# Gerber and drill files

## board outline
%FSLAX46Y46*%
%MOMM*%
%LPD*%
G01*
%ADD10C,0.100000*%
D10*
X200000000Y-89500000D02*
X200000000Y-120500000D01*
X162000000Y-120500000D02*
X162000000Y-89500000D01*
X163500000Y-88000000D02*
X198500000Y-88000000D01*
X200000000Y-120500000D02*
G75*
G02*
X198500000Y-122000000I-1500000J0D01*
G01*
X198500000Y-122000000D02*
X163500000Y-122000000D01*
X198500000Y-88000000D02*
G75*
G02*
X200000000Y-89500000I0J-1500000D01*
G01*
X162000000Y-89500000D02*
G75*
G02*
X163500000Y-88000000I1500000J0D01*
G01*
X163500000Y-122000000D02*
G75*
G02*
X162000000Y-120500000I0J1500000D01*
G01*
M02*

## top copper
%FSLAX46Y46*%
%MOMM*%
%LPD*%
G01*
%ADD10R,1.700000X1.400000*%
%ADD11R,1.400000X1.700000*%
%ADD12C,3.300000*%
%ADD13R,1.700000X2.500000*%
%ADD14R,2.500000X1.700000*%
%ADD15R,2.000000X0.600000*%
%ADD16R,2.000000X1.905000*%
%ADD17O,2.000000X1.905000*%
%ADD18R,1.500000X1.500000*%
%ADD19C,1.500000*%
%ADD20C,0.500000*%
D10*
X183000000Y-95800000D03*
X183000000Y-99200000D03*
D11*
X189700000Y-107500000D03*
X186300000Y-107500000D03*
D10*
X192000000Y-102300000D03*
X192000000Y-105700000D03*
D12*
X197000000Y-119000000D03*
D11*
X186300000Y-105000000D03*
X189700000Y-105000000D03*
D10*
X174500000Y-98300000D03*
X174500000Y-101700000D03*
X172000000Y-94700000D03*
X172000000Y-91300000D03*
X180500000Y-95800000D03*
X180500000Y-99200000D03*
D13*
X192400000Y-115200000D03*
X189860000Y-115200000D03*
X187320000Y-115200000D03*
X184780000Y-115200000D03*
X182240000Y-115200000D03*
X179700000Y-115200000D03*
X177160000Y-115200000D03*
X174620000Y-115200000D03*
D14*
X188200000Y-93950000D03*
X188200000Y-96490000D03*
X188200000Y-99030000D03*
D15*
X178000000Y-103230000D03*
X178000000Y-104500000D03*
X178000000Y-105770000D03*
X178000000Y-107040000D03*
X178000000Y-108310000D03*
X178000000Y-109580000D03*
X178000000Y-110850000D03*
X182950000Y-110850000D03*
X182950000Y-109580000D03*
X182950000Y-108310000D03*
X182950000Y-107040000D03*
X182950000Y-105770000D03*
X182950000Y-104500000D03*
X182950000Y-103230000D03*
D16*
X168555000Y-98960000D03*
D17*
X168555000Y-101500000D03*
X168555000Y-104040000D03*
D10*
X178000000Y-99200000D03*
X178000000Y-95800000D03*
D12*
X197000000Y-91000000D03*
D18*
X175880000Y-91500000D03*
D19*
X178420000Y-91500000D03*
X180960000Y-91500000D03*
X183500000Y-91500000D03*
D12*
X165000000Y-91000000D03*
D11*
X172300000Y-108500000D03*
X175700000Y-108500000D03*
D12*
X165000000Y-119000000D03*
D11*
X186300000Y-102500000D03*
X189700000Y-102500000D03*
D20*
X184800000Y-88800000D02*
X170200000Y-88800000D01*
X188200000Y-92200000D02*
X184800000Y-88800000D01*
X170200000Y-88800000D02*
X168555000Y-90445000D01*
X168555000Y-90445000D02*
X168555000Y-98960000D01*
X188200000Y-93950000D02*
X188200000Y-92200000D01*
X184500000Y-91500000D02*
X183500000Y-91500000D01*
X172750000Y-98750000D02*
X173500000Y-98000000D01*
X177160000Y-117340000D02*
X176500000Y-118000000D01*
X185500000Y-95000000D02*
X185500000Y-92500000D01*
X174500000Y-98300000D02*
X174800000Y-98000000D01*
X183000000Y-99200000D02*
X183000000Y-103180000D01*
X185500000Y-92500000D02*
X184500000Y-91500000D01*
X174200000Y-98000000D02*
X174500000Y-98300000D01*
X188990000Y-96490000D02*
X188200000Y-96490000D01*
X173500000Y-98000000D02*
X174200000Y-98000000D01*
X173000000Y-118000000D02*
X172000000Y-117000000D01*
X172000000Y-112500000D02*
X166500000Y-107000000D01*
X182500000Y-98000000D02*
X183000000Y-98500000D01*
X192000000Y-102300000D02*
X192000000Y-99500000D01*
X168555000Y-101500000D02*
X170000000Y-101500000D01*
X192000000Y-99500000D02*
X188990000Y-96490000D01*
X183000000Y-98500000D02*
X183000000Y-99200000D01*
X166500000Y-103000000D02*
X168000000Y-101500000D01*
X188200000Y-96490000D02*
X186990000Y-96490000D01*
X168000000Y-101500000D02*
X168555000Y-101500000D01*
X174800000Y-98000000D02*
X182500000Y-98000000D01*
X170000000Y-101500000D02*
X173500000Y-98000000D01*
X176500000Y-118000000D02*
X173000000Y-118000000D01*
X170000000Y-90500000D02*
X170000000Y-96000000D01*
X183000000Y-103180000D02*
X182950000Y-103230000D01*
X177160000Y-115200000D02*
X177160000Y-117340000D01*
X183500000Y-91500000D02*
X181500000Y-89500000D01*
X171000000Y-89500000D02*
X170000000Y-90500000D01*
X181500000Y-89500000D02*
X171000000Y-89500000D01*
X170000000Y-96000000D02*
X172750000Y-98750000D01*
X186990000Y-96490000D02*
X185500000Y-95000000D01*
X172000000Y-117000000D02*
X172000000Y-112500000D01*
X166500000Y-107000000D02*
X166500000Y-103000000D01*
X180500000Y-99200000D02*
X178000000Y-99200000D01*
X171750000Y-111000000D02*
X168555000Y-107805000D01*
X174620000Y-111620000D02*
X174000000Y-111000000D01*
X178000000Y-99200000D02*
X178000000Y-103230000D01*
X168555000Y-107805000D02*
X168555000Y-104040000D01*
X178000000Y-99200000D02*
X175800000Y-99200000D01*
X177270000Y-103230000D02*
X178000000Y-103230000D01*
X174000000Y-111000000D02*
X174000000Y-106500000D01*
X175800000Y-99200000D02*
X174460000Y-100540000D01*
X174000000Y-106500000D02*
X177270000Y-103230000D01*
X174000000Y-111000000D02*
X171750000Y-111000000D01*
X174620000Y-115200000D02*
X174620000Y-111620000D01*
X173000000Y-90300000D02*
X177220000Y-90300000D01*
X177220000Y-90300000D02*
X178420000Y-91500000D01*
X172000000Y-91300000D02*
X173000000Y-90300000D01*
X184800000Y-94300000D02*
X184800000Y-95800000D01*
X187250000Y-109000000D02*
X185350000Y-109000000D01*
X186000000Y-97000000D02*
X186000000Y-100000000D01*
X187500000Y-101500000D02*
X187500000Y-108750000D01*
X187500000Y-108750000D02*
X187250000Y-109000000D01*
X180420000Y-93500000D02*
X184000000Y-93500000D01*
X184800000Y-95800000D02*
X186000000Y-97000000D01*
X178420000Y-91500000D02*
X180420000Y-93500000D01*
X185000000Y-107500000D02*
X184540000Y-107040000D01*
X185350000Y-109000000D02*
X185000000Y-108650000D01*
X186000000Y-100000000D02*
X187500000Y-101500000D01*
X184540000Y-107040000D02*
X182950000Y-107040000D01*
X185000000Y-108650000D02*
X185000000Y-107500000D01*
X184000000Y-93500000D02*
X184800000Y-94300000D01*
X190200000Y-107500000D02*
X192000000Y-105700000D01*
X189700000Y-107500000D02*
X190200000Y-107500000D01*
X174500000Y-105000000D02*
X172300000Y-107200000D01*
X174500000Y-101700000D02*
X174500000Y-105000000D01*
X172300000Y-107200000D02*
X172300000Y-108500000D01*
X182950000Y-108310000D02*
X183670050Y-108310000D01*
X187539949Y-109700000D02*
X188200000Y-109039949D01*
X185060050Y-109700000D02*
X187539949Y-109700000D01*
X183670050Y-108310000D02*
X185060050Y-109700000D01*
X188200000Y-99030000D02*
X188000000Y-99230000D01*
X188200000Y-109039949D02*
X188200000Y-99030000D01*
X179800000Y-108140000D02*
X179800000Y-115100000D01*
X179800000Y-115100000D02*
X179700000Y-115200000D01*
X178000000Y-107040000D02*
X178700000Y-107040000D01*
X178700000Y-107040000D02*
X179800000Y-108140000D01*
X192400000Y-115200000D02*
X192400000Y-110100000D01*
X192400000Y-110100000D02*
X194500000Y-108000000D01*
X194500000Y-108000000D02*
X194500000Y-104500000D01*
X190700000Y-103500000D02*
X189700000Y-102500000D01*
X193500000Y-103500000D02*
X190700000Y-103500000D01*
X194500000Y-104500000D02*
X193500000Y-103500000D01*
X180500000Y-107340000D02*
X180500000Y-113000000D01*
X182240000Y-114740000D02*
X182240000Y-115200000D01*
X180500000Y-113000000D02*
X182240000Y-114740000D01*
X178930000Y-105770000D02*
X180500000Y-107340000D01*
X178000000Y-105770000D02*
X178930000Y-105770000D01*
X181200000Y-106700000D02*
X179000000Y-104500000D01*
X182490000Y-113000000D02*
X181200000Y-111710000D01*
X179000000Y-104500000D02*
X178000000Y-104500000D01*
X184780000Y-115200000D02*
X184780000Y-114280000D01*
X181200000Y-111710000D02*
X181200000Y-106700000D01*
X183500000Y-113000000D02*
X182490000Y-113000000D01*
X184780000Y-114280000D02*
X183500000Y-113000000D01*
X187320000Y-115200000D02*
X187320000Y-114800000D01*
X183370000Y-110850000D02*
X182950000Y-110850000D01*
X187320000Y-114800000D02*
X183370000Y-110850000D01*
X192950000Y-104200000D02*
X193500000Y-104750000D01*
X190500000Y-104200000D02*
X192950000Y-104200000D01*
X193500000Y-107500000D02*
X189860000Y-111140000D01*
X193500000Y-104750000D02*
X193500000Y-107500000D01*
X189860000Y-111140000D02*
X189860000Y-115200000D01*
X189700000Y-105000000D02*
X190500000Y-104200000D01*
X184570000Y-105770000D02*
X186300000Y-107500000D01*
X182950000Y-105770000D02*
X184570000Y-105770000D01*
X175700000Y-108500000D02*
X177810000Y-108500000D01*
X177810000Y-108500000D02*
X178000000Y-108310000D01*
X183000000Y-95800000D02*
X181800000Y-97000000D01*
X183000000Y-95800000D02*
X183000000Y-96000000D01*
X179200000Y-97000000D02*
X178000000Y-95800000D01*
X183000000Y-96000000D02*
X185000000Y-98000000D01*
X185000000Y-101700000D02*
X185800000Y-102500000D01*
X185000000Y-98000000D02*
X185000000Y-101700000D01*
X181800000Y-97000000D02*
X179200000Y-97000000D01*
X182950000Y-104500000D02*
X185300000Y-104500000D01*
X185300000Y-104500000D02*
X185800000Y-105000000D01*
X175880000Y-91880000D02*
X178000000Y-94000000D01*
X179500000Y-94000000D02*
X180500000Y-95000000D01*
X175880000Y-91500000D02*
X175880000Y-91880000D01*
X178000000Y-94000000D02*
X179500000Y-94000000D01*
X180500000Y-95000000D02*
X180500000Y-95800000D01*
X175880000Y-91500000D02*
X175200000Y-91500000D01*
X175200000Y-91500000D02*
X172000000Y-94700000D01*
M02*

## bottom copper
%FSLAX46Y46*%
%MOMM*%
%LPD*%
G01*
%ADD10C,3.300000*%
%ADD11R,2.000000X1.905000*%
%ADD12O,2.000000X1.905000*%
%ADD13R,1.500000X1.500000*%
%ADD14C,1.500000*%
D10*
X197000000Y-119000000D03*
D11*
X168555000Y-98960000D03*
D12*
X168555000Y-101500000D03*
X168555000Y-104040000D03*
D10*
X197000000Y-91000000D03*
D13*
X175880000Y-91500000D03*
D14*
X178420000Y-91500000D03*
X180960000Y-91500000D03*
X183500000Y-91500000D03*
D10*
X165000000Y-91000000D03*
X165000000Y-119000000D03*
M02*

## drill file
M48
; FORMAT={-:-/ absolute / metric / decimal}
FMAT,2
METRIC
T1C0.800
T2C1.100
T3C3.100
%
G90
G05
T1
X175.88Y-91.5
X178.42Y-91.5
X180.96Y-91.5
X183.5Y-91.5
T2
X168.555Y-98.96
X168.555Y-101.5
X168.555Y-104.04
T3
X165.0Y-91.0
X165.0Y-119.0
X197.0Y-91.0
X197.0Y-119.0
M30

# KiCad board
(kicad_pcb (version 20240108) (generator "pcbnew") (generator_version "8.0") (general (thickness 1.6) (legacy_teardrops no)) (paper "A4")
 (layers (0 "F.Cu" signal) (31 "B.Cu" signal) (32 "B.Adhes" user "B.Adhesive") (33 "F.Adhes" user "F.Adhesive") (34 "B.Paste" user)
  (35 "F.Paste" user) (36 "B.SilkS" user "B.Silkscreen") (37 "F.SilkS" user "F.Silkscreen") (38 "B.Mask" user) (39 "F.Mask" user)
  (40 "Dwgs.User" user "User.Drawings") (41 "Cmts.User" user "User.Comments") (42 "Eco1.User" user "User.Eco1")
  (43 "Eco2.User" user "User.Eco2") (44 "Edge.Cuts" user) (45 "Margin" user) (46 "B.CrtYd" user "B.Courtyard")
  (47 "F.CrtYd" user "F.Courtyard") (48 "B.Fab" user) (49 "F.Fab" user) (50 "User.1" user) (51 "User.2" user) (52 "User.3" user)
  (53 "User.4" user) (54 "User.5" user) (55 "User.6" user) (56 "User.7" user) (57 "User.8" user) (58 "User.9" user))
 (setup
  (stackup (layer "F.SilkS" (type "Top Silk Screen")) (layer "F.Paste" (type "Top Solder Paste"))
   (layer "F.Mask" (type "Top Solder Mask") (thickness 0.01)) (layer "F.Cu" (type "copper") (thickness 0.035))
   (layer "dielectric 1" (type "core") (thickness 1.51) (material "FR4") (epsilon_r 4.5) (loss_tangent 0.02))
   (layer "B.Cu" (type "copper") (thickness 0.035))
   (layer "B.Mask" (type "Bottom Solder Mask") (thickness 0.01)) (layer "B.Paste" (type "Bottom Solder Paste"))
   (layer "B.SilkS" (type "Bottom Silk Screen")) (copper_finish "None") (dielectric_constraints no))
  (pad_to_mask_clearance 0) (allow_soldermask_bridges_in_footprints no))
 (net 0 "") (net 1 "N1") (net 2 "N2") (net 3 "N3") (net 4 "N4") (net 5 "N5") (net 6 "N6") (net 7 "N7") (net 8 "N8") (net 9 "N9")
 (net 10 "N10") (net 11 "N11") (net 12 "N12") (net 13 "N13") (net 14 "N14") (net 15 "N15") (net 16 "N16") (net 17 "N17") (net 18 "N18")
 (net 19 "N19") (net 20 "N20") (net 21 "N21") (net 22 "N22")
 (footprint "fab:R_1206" (layer "F.Cu") (at 183 97.5 -90)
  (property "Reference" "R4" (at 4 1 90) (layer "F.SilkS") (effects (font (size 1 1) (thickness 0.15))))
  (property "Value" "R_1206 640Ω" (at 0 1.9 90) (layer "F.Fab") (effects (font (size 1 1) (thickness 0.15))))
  (pad "1" smd rect (at -1.7 0 270) (size 1.4 1.7) (layers "F.Cu" "F.Paste" "F.Mask") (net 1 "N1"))
  (pad "2" smd rect (at 1.7 0 270) (size 1.4 1.7) (layers "F.Cu" "F.Paste" "F.Mask") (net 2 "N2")))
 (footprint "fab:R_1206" (layer "F.Cu") (at 188 107.5 180)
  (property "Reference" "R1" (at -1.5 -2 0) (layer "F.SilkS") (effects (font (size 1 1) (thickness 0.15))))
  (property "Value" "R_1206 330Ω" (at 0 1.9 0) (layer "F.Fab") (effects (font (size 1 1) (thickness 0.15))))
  (pad "1" smd rect (at -1.7 0 180) (size 1.4 1.7) (layers "F.Cu" "F.Paste" "F.Mask") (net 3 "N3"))
  (pad "2" smd rect (at 1.7 0 180) (size 1.4 1.7) (layers "F.Cu" "F.Paste" "F.Mask") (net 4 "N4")))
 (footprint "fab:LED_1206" (layer "F.Cu") (at 192 104 -90)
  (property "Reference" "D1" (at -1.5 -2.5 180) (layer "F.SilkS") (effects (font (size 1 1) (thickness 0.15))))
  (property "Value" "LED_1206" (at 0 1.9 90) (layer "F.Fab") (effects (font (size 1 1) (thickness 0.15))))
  (pad "1" smd rect (at -1.7 0 270) (size 1.4 1.7) (layers "F.Cu" "F.Paste" "F.Mask") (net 2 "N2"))
  (pad "2" smd rect (at 1.7 0 270) (size 1.4 1.7) (layers "F.Cu" "F.Paste" "F.Mask") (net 3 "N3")))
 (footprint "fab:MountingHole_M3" (layer "F.Cu") (at 197 119)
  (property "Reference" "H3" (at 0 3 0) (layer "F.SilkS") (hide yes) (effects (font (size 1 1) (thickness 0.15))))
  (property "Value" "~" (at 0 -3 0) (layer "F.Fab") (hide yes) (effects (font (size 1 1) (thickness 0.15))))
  (pad "" thru_hole circle (at 0 0) (size 3.3 3.3) (drill 3.1) (layers "*.Cu" "*.Mask") (remove_unused_layers no)))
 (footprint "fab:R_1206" (layer "F.Cu") (at 188 105)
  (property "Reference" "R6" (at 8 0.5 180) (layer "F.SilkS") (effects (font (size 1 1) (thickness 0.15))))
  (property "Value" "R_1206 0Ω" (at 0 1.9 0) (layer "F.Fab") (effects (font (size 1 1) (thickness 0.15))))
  (pad "1" smd rect (at -1.7 0) (size 1.4 1.7) (layers "F.Cu" "F.Paste" "F.Mask") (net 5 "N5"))
  (pad "2" smd rect (at 1.7 0) (size 1.4 1.7) (layers "F.Cu" "F.Paste" "F.Mask") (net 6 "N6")))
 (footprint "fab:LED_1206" (layer "F.Cu") (at 174.5 100 -90)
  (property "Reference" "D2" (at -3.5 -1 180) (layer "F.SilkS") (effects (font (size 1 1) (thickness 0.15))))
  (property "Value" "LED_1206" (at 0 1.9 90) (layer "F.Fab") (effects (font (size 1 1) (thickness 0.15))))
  (pad "1" smd rect (at -1.7 0 270) (size 1.4 1.7) (layers "F.Cu" "F.Paste" "F.Mask") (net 2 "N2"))
  (pad "2" smd rect (at 1.7 0 270) (size 1.4 1.7) (layers "F.Cu" "F.Paste" "F.Mask") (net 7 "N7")))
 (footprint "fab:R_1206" (layer "F.Cu") (at 172 93 90)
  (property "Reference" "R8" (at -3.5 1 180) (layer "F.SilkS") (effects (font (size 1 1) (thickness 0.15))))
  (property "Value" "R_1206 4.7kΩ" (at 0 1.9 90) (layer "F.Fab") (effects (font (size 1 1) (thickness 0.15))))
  (pad "1" smd rect (at -1.7 0 90) (size 1.4 1.7) (layers "F.Cu" "F.Paste" "F.Mask") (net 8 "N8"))
  (pad "2" smd rect (at 1.7 0 90) (size 1.4 1.7) (layers "F.Cu" "F.Paste" "F.Mask") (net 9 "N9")))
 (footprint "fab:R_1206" (layer "F.Cu") (at 180.5 97.5 -90)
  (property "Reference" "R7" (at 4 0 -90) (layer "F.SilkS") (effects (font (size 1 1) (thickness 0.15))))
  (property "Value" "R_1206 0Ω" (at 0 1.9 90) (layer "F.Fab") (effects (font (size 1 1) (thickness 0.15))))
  (pad "1" smd rect (at -1.7 0 270) (size 1.4 1.7) (layers "F.Cu" "F.Paste" "F.Mask") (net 8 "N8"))
  (pad "2" smd rect (at 1.7 0 270) (size 1.4 1.7) (layers "F.Cu" "F.Paste" "F.Mask") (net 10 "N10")))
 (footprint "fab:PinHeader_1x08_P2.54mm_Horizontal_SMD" (layer "F.Cu") (at 192.4 115.2 -90)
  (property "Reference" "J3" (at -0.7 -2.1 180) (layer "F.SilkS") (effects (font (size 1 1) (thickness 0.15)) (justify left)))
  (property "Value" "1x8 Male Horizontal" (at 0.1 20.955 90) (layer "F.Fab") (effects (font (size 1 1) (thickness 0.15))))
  (pad "1" smd rect (at 0 0 270) (size 2.5 1.7) (layers "F.Cu" "F.Paste" "F.Mask") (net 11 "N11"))
  (pad "2" smd rect (at 0 2.54 270) (size 2.5 1.7) (layers "F.Cu" "F.Paste" "F.Mask") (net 6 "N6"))
  (pad "3" smd rect (at 0 5.08 270) (size 2.5 1.7) (layers "F.Cu" "F.Paste" "F.Mask") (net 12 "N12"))
  (pad "4" smd rect (at 0 7.62 270) (size 2.5 1.7) (layers "F.Cu" "F.Paste" "F.Mask") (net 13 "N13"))
  (pad "5" smd rect (at 0 10.16 270) (size 2.5 1.7) (layers "F.Cu" "F.Paste" "F.Mask") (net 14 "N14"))
  (pad "6" smd rect (at 0 12.7 270) (size 2.5 1.7) (layers "F.Cu" "F.Paste" "F.Mask") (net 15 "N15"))
  (pad "7" smd rect (at 0 15.24 270) (size 2.5 1.7) (layers "F.Cu" "F.Paste" "F.Mask") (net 2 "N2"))
  (pad "8" smd rect (at 0 17.78 270) (size 2.5 1.7) (layers "F.Cu" "F.Paste" "F.Mask") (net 10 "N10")))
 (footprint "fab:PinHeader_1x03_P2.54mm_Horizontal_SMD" (layer "F.Cu") (at 188.2 93.95)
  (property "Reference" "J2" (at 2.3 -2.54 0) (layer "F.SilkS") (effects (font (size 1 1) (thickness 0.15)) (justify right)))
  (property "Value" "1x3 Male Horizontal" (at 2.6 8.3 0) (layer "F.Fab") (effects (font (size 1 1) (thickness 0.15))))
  (pad "1" smd rect (at 0 0) (size 2.5 1.7) (layers "F.Cu" "F.Paste" "F.Mask") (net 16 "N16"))
  (pad "2" smd rect (at 0 2.54) (size 2.5 1.7) (layers "F.Cu" "F.Paste" "F.Mask") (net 2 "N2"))
  (pad "3" smd rect (at 0 5.08) (size 2.5 1.7) (layers "F.Cu" "F.Paste" "F.Mask") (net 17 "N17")))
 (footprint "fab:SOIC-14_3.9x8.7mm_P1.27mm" (layer "F.Cu") (at 180.475 107.04)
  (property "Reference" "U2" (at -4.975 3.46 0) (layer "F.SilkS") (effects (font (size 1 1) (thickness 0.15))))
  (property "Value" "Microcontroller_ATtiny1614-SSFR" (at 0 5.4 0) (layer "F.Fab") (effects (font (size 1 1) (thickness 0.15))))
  (pad "1" smd rect (at -2.475 -3.81) (size 2 0.6) (layers "F.Cu" "F.Paste" "F.Mask") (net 10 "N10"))
  (pad "2" smd rect (at -2.475 -2.54) (size 2 0.6) (layers "F.Cu" "F.Paste" "F.Mask") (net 13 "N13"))
  (pad "3" smd rect (at -2.475 -1.27) (size 2 0.6) (layers "F.Cu" "F.Paste" "F.Mask") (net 14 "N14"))
  (pad "4" smd rect (at -2.475 0) (size 2 0.6) (layers "F.Cu" "F.Paste" "F.Mask") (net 15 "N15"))
  (pad "5" smd rect (at -2.475 1.27) (size 2 0.6) (layers "F.Cu" "F.Paste" "F.Mask") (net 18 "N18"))
  (pad "6" smd rect (at -2.475 2.54) (size 2 0.6) (layers "F.Cu" "F.Paste" "F.Mask") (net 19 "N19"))
  (pad "7" smd rect (at -2.475 3.81) (size 2 0.6) (layers "F.Cu" "F.Paste" "F.Mask") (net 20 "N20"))
  (pad "8" smd rect (at 2.475 3.81) (size 2 0.6) (layers "F.Cu" "F.Paste" "F.Mask") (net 12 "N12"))
  (pad "9" smd rect (at 2.475 2.54) (size 2 0.6) (layers "F.Cu" "F.Paste" "F.Mask") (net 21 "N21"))
  (pad "10" smd rect (at 2.475 1.27) (size 2 0.6) (layers "F.Cu" "F.Paste" "F.Mask") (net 17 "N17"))
  (pad "11" smd rect (at 2.475 0) (size 2 0.6) (layers "F.Cu" "F.Paste" "F.Mask") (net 9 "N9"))
  (pad "12" smd rect (at 2.475 -1.27) (size 2 0.6) (layers "F.Cu" "F.Paste" "F.Mask") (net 4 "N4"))
  (pad "13" smd rect (at 2.475 -2.54) (size 2 0.6) (layers "F.Cu" "F.Paste" "F.Mask") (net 5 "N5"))
  (pad "14" smd rect (at 2.475 -3.81) (size 2 0.6) (layers "F.Cu" "F.Paste" "F.Mask") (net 2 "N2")))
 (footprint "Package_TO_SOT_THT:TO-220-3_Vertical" (layer "F.Cu") (at 168.555 98.96 -90)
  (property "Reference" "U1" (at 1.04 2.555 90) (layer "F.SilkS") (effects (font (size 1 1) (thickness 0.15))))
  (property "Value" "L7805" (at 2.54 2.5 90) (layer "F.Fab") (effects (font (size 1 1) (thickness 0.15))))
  (pad "1" thru_hole rect (at 0 0 270) (size 1.905 2) (drill 1.1) (layers "*.Cu" "*.Mask") (remove_unused_layers no) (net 16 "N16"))
  (pad "2" thru_hole oval (at 2.54 0 270) (size 1.905 2) (drill 1.1) (layers "*.Cu" "*.Mask") (remove_unused_layers no) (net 2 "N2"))
  (pad "3" thru_hole oval (at 5.08 0 270) (size 1.905 2) (drill 1.1) (layers "*.Cu" "*.Mask") (remove_unused_layers no) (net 10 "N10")))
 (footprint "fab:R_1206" (layer "F.Cu") (at 178 97.5 90)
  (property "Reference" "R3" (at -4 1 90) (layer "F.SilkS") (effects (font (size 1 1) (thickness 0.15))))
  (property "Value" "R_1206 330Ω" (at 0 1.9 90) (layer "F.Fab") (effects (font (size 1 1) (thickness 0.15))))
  (pad "1" smd rect (at -1.7 0 90) (size 1.4 1.7) (layers "F.Cu" "F.Paste" "F.Mask") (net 10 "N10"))
  (pad "2" smd rect (at 1.7 0 90) (size 1.4 1.7) (layers "F.Cu" "F.Paste" "F.Mask") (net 1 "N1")))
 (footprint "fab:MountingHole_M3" (layer "F.Cu") (at 197 91)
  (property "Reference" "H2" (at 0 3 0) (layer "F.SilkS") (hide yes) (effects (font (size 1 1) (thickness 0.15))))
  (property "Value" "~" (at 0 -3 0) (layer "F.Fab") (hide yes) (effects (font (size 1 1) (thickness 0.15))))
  (pad "" thru_hole circle (at 0 0) (size 3.3 3.3) (drill 3.1) (layers "*.Cu" "*.Mask") (remove_unused_layers no)))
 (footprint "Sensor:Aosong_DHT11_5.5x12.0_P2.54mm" (layer "F.Cu") (at 175.88 91.5 90)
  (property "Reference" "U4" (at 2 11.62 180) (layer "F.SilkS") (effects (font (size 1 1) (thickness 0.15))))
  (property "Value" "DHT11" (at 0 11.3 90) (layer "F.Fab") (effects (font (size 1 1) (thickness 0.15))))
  (pad "1" thru_hole rect (at 0 0 90) (size 1.5 1.5) (drill 0.8) (layers "*.Cu" "*.Mask") (remove_unused_layers no) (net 8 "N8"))
  (pad "2" thru_hole circle (at 0 2.54 90) (size 1.5 1.5) (drill 0.8) (layers "*.Cu" "*.Mask") (remove_unused_layers no) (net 9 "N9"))
  (pad "3" thru_hole circle (at 0 5.08 90) (size 1.5 1.5) (drill 0.8) (layers "*.Cu" "*.Mask") (remove_unused_layers no) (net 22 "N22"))
  (pad "4" thru_hole circle (at 0 7.62 90) (size 1.5 1.5) (drill 0.8) (layers "*.Cu" "*.Mask") (remove_unused_layers no) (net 2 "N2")))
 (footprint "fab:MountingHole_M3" (layer "F.Cu") (at 165 91)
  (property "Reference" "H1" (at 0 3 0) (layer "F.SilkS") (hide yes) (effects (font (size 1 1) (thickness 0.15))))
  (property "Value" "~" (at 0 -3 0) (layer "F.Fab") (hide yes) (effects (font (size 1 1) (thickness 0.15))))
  (pad "" thru_hole circle (at 0 0) (size 3.3 3.3) (drill 3.1) (layers "*.Cu" "*.Mask") (remove_unused_layers no)))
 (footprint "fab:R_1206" (layer "F.Cu") (at 174 108.5)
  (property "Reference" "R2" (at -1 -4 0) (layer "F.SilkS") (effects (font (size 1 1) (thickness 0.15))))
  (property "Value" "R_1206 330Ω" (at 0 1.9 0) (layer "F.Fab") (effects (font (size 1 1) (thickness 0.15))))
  (pad "1" smd rect (at -1.7 0) (size 1.4 1.7) (layers "F.Cu" "F.Paste" "F.Mask") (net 7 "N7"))
  (pad "2" smd rect (at 1.7 0) (size 1.4 1.7) (layers "F.Cu" "F.Paste" "F.Mask") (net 18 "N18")))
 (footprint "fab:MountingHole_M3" (layer "F.Cu") (at 165 119)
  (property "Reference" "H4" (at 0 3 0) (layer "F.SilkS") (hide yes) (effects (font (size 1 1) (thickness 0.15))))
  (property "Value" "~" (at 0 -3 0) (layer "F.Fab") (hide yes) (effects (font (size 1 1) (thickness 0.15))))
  (pad "" thru_hole circle (at 0 0) (size 3.3 3.3) (drill 3.1) (layers "*.Cu" "*.Mask") (remove_unused_layers no)))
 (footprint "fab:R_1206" (layer "F.Cu") (at 188 102.5)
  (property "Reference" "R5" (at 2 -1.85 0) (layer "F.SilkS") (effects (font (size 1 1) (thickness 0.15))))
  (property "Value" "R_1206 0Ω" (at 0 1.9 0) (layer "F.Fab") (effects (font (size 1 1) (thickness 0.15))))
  (pad "1" smd rect (at -1.7 0) (size 1.4 1.7) (layers "F.Cu" "F.Paste" "F.Mask") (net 1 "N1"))
  (pad "2" smd rect (at 1.7 0) (size 1.4 1.7) (layers "F.Cu" "F.Paste" "F.Mask") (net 11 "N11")))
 (gr_line (start 200 89.5) (end 200 120.5) (stroke (width 0.1) (type default)) (layer "Edge.Cuts"))
 (gr_line (start 162 120.5) (end 162 89.5) (stroke (width 0.1) (type default)) (layer "Edge.Cuts"))
 (gr_line (start 163.5 88) (end 198.5 88) (stroke (width 0.1) (type default)) (layer "Edge.Cuts"))
 (gr_arc (start 200 120.5) (mid 199.56066 121.56066) (end 198.5 122) (stroke (width 0.1) (type default)) (layer "Edge.Cuts"))
 (gr_line (start 198.5 122) (end 163.5 122) (stroke (width 0.1) (type default)) (layer "Edge.Cuts"))
 (gr_arc (start 198.5 88) (mid 199.56066 88.43934) (end 200 89.5) (stroke (width 0.1) (type default)) (layer "Edge.Cuts"))
 (gr_arc (start 162 89.5) (mid 162.43934 88.43934) (end 163.5 88) (stroke (width 0.1) (type default)) (layer "Edge.Cuts"))
 (gr_arc (start 163.5 122) (mid 162.43934 121.56066) (end 162 120.5) (stroke (width 0.1) (type default)) (layer "Edge.Cuts"))
 (segment (start 184.8 88.8) (end 170.2 88.8) (width 0.5) (layer "F.Cu") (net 16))
 (segment (start 188.2 92.2) (end 184.8 88.8) (width 0.5) (layer "F.Cu") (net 16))
 (segment (start 170.2 88.8) (end 168.555 90.445) (width 0.5) (layer "F.Cu") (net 16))
 (segment (start 168.555 90.445) (end 168.555 98.96) (width 0.5) (layer "F.Cu") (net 16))
 (segment (start 188.2 93.95) (end 188.2 92.2) (width 0.5) (layer "F.Cu") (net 16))
 (segment (start 184.5 91.5) (end 183.5 91.5) (width 0.5) (layer "F.Cu") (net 2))
 (segment (start 172.75 98.75) (end 173.5 98) (width 0.5) (layer "F.Cu") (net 2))
 (segment (start 177.16 117.34) (end 176.5 118) (width 0.5) (layer "F.Cu") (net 2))
 (segment (start 185.5 95) (end 185.5 92.5) (width 0.5) (layer "F.Cu") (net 2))
 (segment (start 174.5 98.3) (end 174.8 98) (width 0.5) (layer "F.Cu") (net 2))
 (segment (start 183 99.2) (end 183 103.18) (width 0.5) (layer "F.Cu") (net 2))
 (segment (start 185.5 92.5) (end 184.5 91.5) (width 0.5) (layer "F.Cu") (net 2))
 (segment (start 174.2 98) (end 174.5 98.3) (width 0.5) (layer "F.Cu") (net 2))
 (segment (start 188.99 96.49) (end 188.2 96.49) (width 0.5) (layer "F.Cu") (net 2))
 (segment (start 173.5 98) (end 174.2 98) (width 0.5) (layer "F.Cu") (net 2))
 (segment (start 173 118) (end 172 117) (width 0.5) (layer "F.Cu") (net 2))
 (segment (start 172 112.5) (end 166.5 107) (width 0.5) (layer "F.Cu") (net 2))
 (segment (start 182.5 98) (end 183 98.5) (width 0.5) (layer "F.Cu") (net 2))
 (segment (start 192 102.3) (end 192 99.5) (width 0.5) (layer "F.Cu") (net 2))
 (segment (start 168.555 101.5) (end 170 101.5) (width 0.5) (layer "F.Cu") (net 2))
 (segment (start 192 99.5) (end 188.99 96.49) (width 0.5) (layer "F.Cu") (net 2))
 (segment (start 183 98.5) (end 183 99.2) (width 0.5) (layer "F.Cu") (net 2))
 (segment (start 166.5 103) (end 168 101.5) (width 0.5) (layer "F.Cu") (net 2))
 (segment (start 188.2 96.49) (end 186.99 96.49) (width 0.5) (layer "F.Cu") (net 2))
 (segment (start 168 101.5) (end 168.555 101.5) (width 0.5) (layer "F.Cu") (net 2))
 (segment (start 174.8 98) (end 182.5 98) (width 0.5) (layer "F.Cu") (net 2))
 (segment (start 170 101.5) (end 173.5 98) (width 0.5) (layer "F.Cu") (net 2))
 (segment (start 176.5 118) (end 173 118) (width 0.5) (layer "F.Cu") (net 2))
 (segment (start 170 90.5) (end 170 96) (width 0.5) (layer "F.Cu") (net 2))
 (segment (start 183 103.18) (end 182.95 103.23) (width 0.5) (layer "F.Cu") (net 2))
 (segment (start 177.16 115.2) (end 177.16 117.34) (width 0.5) (layer "F.Cu") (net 2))
 (segment (start 183.5 91.5) (end 181.5 89.5) (width 0.5) (layer "F.Cu") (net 2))
 (segment (start 171 89.5) (end 170 90.5) (width 0.5) (layer "F.Cu") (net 2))
 (segment (start 181.5 89.5) (end 171 89.5) (width 0.5) (layer "F.Cu") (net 2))
 (segment (start 170 96) (end 172.75 98.75) (width 0.5) (layer "F.Cu") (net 2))
 (segment (start 186.99 96.49) (end 185.5 95) (width 0.5) (layer "F.Cu") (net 2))
 (segment (start 172 117) (end 172 112.5) (width 0.5) (layer "F.Cu") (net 2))
 (segment (start 166.5 107) (end 166.5 103) (width 0.5) (layer "F.Cu") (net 2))
 (segment (start 180.5 99.2) (end 178 99.2) (width 0.5) (layer "F.Cu") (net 10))
 (segment (start 171.75 111) (end 168.555 107.805) (width 0.5) (layer "F.Cu") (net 10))
 (segment (start 174.62 111.62) (end 174 111) (width 0.5) (layer "F.Cu") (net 10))
 (segment (start 178 99.2) (end 178 103.23) (width 0.5) (layer "F.Cu") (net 10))
 (segment (start 168.555 107.805) (end 168.555 104.04) (width 0.5) (layer "F.Cu") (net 10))
 (segment (start 178 99.2) (end 175.8 99.2) (width 0.5) (layer "F.Cu") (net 10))
 (segment (start 177.27 103.23) (end 178 103.23) (width 0.5) (layer "F.Cu") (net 10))
 (segment (start 174 111) (end 174 106.5) (width 0.5) (layer "F.Cu") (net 10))
 (segment (start 175.8 99.2) (end 174.46 100.54) (width 0.5) (layer "F.Cu") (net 10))
 (segment (start 174 106.5) (end 177.27 103.23) (width 0.5) (layer "F.Cu") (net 10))
 (segment (start 174 111) (end 171.75 111) (width 0.5) (layer "F.Cu") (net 10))
 (segment (start 174.62 115.2) (end 174.62 111.62) (width 0.5) (layer "F.Cu") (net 10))
 (segment (start 173 90.3) (end 177.22 90.3) (width 0.5) (layer "F.Cu") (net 9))
 (segment (start 177.22 90.3) (end 178.42 91.5) (width 0.5) (layer "F.Cu") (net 9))
 (segment (start 172 91.3) (end 173 90.3) (width 0.5) (layer "F.Cu") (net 9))
 (segment (start 184.8 94.3) (end 184.8 95.8) (width 0.5) (layer "F.Cu") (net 9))
 (segment (start 187.25 109) (end 185.35 109) (width 0.5) (layer "F.Cu") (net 9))
 (segment (start 186 97) (end 186 100) (width 0.5) (layer "F.Cu") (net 9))
 (segment (start 187.5 101.5) (end 187.5 108.75) (width 0.5) (layer "F.Cu") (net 9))
 (segment (start 187.5 108.75) (end 187.25 109) (width 0.5) (layer "F.Cu") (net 9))
 (segment (start 180.42 93.5) (end 184 93.5) (width 0.5) (layer "F.Cu") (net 9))
 (segment (start 184.8 95.8) (end 186 97) (width 0.5) (layer "F.Cu") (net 9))
 (segment (start 178.42 91.5) (end 180.42 93.5) (width 0.5) (layer "F.Cu") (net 9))
 (segment (start 185 107.5) (end 184.54 107.04) (width 0.5) (layer "F.Cu") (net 9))
 (segment (start 185.35 109) (end 185 108.65) (width 0.5) (layer "F.Cu") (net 9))
 (segment (start 186 100) (end 187.5 101.5) (width 0.5) (layer "F.Cu") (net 9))
 (segment (start 184.54 107.04) (end 182.95 107.04) (width 0.5) (layer "F.Cu") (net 9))
 (segment (start 185 108.65) (end 185 107.5) (width 0.5) (layer "F.Cu") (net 9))
 (segment (start 184 93.5) (end 184.8 94.3) (width 0.5) (layer "F.Cu") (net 9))
 (segment (start 190.2 107.5) (end 192 105.7) (width 0.5) (layer "F.Cu") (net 3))
 (segment (start 189.7 107.5) (end 190.2 107.5) (width 0.5) (layer "F.Cu") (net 3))
 (segment (start 174.5 105) (end 172.3 107.2) (width 0.5) (layer "F.Cu") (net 7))
 (segment (start 174.5 101.7) (end 174.5 105) (width 0.5) (layer "F.Cu") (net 7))
 (segment (start 172.3 107.2) (end 172.3 108.5) (width 0.5) (layer "F.Cu") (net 7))
 (segment (start 182.95 108.31) (end 183.67005 108.31) (width 0.5) (layer "F.Cu") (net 17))
 (segment (start 187.539949 109.7) (end 188.2 109.039949) (width 0.5) (layer "F.Cu") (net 17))
 (segment (start 185.06005 109.7) (end 187.539949 109.7) (width 0.5) (layer "F.Cu") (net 17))
 (segment (start 183.67005 108.31) (end 185.06005 109.7) (width 0.5) (layer "F.Cu") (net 17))
 (segment (start 188.2 99.03) (end 188 99.23) (width 0.5) (layer "F.Cu") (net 17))
 (segment (start 188.2 109.039949) (end 188.2 99.03) (width 0.5) (layer "F.Cu") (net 17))
 (segment (start 179.8 108.14) (end 179.8 115.1) (width 0.5) (layer "F.Cu") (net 15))
 (segment (start 179.8 115.1) (end 179.7 115.2) (width 0.5) (layer "F.Cu") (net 15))
 (segment (start 178 107.04) (end 178.7 107.04) (width 0.5) (layer "F.Cu") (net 15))
 (segment (start 178.7 107.04) (end 179.8 108.14) (width 0.5) (layer "F.Cu") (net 15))
 (segment (start 192.4 115.2) (end 192.4 110.1) (width 0.5) (layer "F.Cu") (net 11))
 (segment (start 192.4 110.1) (end 194.5 108) (width 0.5) (layer "F.Cu") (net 11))
 (segment (start 194.5 108) (end 194.5 104.5) (width 0.5) (layer "F.Cu") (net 11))
 (segment (start 190.7 103.5) (end 189.7 102.5) (width 0.5) (layer "F.Cu") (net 11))
 (segment (start 193.5 103.5) (end 190.7 103.5) (width 0.5) (layer "F.Cu") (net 11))
 (segment (start 194.5 104.5) (end 193.5 103.5) (width 0.5) (layer "F.Cu") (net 11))
 (segment (start 180.5 107.34) (end 180.5 113) (width 0.5) (layer "F.Cu") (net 14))
 (segment (start 182.24 114.74) (end 182.24 115.2) (width 0.5) (layer "F.Cu") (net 14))
 (segment (start 180.5 113) (end 182.24 114.74) (width 0.5) (layer "F.Cu") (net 14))
 (segment (start 178.93 105.77) (end 180.5 107.34) (width 0.5) (layer "F.Cu") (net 14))
 (segment (start 178 105.77) (end 178.93 105.77) (width 0.5) (layer "F.Cu") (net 14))
 (segment (start 181.2 106.7) (end 179 104.5) (width 0.5) (layer "F.Cu") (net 13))
 (segment (start 182.49 113) (end 181.2 111.71) (width 0.5) (layer "F.Cu") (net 13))
 (segment (start 179 104.5) (end 178 104.5) (width 0.5) (layer "F.Cu") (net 13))
 (segment (start 184.78 115.2) (end 184.78 114.28) (width 0.5) (layer "F.Cu") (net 13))
 (segment (start 181.2 111.71) (end 181.2 106.7) (width 0.5) (layer "F.Cu") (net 13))
 (segment (start 183.5 113) (end 182.49 113) (width 0.5) (layer "F.Cu") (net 13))
 (segment (start 184.78 114.28) (end 183.5 113) (width 0.5) (layer "F.Cu") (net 13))
 (segment (start 187.32 115.2) (end 187.32 114.8) (width 0.5) (layer "F.Cu") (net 12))
 (segment (start 183.37 110.85) (end 182.95 110.85) (width 0.5) (layer "F.Cu") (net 12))
 (segment (start 187.32 114.8) (end 183.37 110.85) (width 0.5) (layer "F.Cu") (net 12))
 (segment (start 192.95 104.2) (end 193.5 104.75) (width 0.5) (layer "F.Cu") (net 6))
 (segment (start 190.5 104.2) (end 192.95 104.2) (width 0.5) (layer "F.Cu") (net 6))
 (segment (start 193.5 107.5) (end 189.86 111.14) (width 0.5) (layer "F.Cu") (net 6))
 (segment (start 193.5 104.75) (end 193.5 107.5) (width 0.5) (layer "F.Cu") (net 6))
 (segment (start 189.86 111.14) (end 189.86 115.2) (width 0.5) (layer "F.Cu") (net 6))
 (segment (start 189.7 105) (end 190.5 104.2) (width 0.5) (layer "F.Cu") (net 6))
 (segment (start 184.57 105.77) (end 186.3 107.5) (width 0.5) (layer "F.Cu") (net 4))
 (segment (start 182.95 105.77) (end 184.57 105.77) (width 0.5) (layer "F.Cu") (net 4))
 (segment (start 175.7 108.5) (end 177.81 108.5) (width 0.5) (layer "F.Cu") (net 18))
 (segment (start 177.81 108.5) (end 178 108.31) (width 0.5) (layer "F.Cu") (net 18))
 (segment (start 183 95.8) (end 181.8 97) (width 0.5) (layer "F.Cu") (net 1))
 (segment (start 183 95.8) (end 183 96) (width 0.5) (layer "F.Cu") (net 1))
 (segment (start 179.2 97) (end 178 95.8) (width 0.5) (layer "F.Cu") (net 1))
 (segment (start 183 96) (end 185 98) (width 0.5) (layer "F.Cu") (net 1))
 (segment (start 185 101.7) (end 185.8 102.5) (width 0.5) (layer "F.Cu") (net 1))
 (segment (start 185 98) (end 185 101.7) (width 0.5) (layer "F.Cu") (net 1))
 (segment (start 181.8 97) (end 179.2 97) (width 0.5) (layer "F.Cu") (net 1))
 (segment (start 182.95 104.5) (end 185.3 104.5) (width 0.5) (layer "F.Cu") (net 5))
 (segment (start 185.3 104.5) (end 185.8 105) (width 0.5) (layer "F.Cu") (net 5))
 (segment (start 175.88 91.88) (end 178 94) (width 0.5) (layer "F.Cu") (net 8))
 (segment (start 179.5 94) (end 180.5 95) (width 0.5) (layer "F.Cu") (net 8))
 (segment (start 175.88 91.5) (end 175.88 91.88) (width 0.5) (layer "F.Cu") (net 8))
 (segment (start 178 94) (end 179.5 94) (width 0.5) (layer "F.Cu") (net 8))
 (segment (start 180.5 95) (end 180.5 95.8) (width 0.5) (layer "F.Cu") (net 8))
 (segment (start 175.88 91.5) (end 175.2 91.5) (width 0.5) (layer "F.Cu") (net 8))
 (segment (start 175.2 91.5) (end 172 94.7) (width 0.5) (layer "F.Cu") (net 8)))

